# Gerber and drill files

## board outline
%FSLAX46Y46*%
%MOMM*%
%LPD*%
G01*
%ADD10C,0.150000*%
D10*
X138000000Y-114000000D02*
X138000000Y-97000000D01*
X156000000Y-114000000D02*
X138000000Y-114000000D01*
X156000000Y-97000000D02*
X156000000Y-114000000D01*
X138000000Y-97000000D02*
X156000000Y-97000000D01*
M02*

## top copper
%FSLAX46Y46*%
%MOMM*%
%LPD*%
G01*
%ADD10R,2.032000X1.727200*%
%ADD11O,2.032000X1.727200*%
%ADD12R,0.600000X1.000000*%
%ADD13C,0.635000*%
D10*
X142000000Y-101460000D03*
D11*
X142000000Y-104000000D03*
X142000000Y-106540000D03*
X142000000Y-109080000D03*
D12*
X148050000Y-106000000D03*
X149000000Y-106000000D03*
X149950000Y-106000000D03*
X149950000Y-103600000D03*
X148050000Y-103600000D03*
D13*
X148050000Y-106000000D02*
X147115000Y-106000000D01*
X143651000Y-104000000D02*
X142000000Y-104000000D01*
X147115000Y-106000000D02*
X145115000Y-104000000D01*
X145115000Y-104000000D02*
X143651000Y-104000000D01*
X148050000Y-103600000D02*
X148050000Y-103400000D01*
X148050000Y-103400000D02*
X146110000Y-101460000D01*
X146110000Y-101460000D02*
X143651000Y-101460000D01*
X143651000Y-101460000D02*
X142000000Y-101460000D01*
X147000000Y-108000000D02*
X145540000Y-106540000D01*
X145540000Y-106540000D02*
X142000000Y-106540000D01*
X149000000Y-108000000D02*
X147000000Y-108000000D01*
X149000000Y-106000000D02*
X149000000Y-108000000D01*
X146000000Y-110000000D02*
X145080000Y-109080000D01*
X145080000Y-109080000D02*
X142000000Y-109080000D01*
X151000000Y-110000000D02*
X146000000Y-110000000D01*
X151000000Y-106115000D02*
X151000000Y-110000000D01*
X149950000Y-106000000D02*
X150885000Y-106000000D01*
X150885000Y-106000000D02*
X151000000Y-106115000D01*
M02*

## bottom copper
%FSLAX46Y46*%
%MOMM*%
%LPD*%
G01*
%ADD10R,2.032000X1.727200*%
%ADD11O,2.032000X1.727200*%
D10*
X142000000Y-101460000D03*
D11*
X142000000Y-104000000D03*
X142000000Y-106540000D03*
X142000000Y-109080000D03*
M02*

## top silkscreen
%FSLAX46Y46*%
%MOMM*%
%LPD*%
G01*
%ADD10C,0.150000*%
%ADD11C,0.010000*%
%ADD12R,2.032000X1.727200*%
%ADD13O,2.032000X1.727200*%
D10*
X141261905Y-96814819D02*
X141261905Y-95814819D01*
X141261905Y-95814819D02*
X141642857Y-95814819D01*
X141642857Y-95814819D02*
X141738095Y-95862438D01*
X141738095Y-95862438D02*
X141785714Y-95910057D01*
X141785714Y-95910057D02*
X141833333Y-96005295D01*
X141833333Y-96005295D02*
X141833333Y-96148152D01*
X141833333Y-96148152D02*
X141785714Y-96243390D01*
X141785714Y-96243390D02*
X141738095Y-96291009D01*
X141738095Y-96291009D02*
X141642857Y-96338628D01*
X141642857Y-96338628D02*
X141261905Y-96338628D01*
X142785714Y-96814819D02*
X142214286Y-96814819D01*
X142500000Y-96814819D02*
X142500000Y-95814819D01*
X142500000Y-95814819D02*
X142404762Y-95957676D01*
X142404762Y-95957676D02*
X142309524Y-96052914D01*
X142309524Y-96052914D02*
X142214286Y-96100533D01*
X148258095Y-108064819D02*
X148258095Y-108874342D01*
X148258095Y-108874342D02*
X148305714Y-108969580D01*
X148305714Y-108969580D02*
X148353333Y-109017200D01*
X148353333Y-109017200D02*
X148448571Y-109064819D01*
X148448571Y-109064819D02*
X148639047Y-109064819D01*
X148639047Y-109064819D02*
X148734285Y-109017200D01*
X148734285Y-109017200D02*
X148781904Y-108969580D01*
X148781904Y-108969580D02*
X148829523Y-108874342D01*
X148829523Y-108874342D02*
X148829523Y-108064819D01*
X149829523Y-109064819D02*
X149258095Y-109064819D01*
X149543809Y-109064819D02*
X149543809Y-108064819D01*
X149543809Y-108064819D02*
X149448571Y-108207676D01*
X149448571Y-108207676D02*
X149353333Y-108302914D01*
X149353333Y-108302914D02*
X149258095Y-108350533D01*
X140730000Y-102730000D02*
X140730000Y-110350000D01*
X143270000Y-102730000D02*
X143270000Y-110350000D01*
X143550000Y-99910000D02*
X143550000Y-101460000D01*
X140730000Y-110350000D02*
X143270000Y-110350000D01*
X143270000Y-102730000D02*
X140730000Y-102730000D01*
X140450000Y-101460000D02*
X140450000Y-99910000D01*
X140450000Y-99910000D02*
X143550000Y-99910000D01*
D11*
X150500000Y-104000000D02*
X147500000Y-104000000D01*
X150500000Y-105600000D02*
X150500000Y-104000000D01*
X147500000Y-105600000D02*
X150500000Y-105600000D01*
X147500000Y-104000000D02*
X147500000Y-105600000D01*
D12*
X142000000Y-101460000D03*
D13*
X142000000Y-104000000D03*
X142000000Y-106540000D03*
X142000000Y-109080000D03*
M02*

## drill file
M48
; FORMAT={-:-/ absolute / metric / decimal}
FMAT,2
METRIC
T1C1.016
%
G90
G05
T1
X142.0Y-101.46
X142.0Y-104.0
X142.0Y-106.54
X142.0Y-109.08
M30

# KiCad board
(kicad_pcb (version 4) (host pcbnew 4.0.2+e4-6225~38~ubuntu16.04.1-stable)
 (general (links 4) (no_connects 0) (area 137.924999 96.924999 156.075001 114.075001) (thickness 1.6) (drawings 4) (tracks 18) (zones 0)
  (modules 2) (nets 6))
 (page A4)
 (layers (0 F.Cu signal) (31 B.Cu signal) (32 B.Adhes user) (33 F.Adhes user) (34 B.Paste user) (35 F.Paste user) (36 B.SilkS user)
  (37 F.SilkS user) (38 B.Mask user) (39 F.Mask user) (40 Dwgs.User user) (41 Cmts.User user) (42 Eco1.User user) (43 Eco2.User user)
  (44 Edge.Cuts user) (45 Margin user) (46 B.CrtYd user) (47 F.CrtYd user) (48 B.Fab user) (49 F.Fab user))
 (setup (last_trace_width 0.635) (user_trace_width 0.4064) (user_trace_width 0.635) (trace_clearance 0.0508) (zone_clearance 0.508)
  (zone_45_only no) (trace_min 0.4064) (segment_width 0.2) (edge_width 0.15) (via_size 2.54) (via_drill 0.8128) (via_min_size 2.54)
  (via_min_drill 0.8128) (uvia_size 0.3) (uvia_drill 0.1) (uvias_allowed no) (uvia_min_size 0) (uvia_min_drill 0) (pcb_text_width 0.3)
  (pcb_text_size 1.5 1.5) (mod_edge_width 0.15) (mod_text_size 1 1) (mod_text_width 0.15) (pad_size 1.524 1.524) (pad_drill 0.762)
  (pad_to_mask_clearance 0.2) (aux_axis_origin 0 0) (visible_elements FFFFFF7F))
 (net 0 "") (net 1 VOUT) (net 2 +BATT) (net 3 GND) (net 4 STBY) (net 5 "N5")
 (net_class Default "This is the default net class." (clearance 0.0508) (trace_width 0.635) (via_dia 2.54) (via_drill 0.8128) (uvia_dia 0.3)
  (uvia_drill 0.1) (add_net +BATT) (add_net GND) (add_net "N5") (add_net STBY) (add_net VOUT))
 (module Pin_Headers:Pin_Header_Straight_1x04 (layer F.Cu) (at 142 101.46)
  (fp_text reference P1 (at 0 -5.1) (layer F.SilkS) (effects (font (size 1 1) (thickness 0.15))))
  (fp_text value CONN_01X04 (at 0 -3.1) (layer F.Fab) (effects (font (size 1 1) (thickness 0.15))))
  (fp_line (start -1.27 1.27) (end -1.27 8.89) (layer F.SilkS) (width 0.15))
  (fp_line (start 1.27 1.27) (end 1.27 8.89) (layer F.SilkS) (width 0.15))
  (fp_line (start 1.55 -1.55) (end 1.55 0) (layer F.SilkS) (width 0.15))
  (fp_line (start -1.27 8.89) (end 1.27 8.89) (layer F.SilkS) (width 0.15))
  (fp_line (start 1.27 1.27) (end -1.27 1.27) (layer F.SilkS) (width 0.15))
  (fp_line (start -1.55 0) (end -1.55 -1.55) (layer F.SilkS) (width 0.15))
  (fp_line (start -1.55 -1.55) (end 1.55 -1.55) (layer F.SilkS) (width 0.15))
  (pad 1 thru_hole rect (at 0 0) (size 2.032 1.7272) (drill 1.016) (layers *.Cu *.Mask F.SilkS) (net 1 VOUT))
  (pad 2 thru_hole oval (at 0 2.54) (size 2.032 1.7272) (drill 1.016) (layers *.Cu *.Mask F.SilkS) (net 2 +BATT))
  (pad 3 thru_hole oval (at 0 5.08) (size 2.032 1.7272) (drill 1.016) (layers *.Cu *.Mask F.SilkS) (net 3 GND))
  (pad 4 thru_hole oval (at 0 7.62) (size 2.032 1.7272) (drill 1.016) (layers *.Cu *.Mask F.SilkS) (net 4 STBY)))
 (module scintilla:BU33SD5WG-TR (layer F.Cu) (at 149 104.8)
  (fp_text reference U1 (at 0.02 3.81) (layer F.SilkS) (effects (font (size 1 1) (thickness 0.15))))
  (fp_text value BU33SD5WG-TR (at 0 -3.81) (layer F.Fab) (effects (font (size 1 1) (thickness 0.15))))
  (fp_line (start 1.5 -0.8) (end -1.5 -0.8) (layer F.SilkS) (width 0.01))
  (fp_line (start 1.5 0.8) (end 1.5 -0.8) (layer F.SilkS) (width 0.01))
  (fp_line (start -1.5 0.8) (end 1.5 0.8) (layer F.SilkS) (width 0.01))
  (fp_line (start -1.5 -0.8) (end -1.5 0.8) (layer F.SilkS) (width 0.01))
  (pad 1 smd rect (at -0.95 1.2) (size 0.6 1) (layers F.Cu F.Paste F.Mask) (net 2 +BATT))
  (pad 2 smd rect (at 0 1.2) (size 0.6 1) (layers F.Cu F.Paste F.Mask) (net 3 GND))
  (pad 3 smd rect (at 0.95 1.2) (size 0.6 1) (layers F.Cu F.Paste F.Mask) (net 4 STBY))
  (pad 4 smd rect (at 0.95 -1.2) (size 0.6 1) (layers F.Cu F.Paste F.Mask) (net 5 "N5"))
  (pad 5 smd rect (at -0.95 -1.2) (size 0.6 1) (layers F.Cu F.Paste F.Mask) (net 1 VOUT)))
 (gr_line (start 138 114) (end 138 97) (layer Edge.Cuts) (width 0.15))
 (gr_line (start 156 114) (end 138 114) (layer Edge.Cuts) (width 0.15))
 (gr_line (start 156 97) (end 156 114) (layer Edge.Cuts) (width 0.15))
 (gr_line (start 138 97) (end 156 97) (layer Edge.Cuts) (width 0.15))
 (segment (start 148.05 106) (end 147.115 106) (width 0.635) (layer F.Cu) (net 2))
 (segment (start 143.651 104) (end 142 104) (width 0.635) (layer F.Cu) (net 2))
 (segment (start 147.115 106) (end 145.115 104) (width 0.635) (layer F.Cu) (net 2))
 (segment (start 145.115 104) (end 143.651 104) (width 0.635) (layer F.Cu) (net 2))
 (segment (start 148.05 103.6) (end 148.05 103.4) (width 0.635) (layer F.Cu) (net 1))
 (segment (start 148.05 103.4) (end 146.11 101.46) (width 0.635) (layer F.Cu) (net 1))
 (segment (start 146.11 101.46) (end 143.651 101.46) (width 0.635) (layer F.Cu) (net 1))
 (segment (start 143.651 101.46) (end 142 101.46) (width 0.635) (layer F.Cu) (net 1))
 (segment (start 147 108) (end 145.54 106.54) (width 0.635) (layer F.Cu) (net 3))
 (segment (start 145.54 106.54) (end 142 106.54) (width 0.635) (layer F.Cu) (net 3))
 (segment (start 149 108) (end 147 108) (width 0.635) (layer F.Cu) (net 3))
 (segment (start 149 106) (end 149 108) (width 0.635) (layer F.Cu) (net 3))
 (segment (start 146 110) (end 145.08 109.08) (width 0.635) (layer F.Cu) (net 4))
 (segment (start 145.08 109.08) (end 142 109.08) (width 0.635) (layer F.Cu) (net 4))
 (segment (start 151 110) (end 146 110) (width 0.635) (layer F.Cu) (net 4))
 (segment (start 151 106.115) (end 151 110) (width 0.635) (layer F.Cu) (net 4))
 (segment (start 149.95 106) (end 150.885 106) (width 0.635) (layer F.Cu) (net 4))
 (segment (start 150.885 106) (end 151 106.115) (width 0.635) (layer F.Cu) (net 4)))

